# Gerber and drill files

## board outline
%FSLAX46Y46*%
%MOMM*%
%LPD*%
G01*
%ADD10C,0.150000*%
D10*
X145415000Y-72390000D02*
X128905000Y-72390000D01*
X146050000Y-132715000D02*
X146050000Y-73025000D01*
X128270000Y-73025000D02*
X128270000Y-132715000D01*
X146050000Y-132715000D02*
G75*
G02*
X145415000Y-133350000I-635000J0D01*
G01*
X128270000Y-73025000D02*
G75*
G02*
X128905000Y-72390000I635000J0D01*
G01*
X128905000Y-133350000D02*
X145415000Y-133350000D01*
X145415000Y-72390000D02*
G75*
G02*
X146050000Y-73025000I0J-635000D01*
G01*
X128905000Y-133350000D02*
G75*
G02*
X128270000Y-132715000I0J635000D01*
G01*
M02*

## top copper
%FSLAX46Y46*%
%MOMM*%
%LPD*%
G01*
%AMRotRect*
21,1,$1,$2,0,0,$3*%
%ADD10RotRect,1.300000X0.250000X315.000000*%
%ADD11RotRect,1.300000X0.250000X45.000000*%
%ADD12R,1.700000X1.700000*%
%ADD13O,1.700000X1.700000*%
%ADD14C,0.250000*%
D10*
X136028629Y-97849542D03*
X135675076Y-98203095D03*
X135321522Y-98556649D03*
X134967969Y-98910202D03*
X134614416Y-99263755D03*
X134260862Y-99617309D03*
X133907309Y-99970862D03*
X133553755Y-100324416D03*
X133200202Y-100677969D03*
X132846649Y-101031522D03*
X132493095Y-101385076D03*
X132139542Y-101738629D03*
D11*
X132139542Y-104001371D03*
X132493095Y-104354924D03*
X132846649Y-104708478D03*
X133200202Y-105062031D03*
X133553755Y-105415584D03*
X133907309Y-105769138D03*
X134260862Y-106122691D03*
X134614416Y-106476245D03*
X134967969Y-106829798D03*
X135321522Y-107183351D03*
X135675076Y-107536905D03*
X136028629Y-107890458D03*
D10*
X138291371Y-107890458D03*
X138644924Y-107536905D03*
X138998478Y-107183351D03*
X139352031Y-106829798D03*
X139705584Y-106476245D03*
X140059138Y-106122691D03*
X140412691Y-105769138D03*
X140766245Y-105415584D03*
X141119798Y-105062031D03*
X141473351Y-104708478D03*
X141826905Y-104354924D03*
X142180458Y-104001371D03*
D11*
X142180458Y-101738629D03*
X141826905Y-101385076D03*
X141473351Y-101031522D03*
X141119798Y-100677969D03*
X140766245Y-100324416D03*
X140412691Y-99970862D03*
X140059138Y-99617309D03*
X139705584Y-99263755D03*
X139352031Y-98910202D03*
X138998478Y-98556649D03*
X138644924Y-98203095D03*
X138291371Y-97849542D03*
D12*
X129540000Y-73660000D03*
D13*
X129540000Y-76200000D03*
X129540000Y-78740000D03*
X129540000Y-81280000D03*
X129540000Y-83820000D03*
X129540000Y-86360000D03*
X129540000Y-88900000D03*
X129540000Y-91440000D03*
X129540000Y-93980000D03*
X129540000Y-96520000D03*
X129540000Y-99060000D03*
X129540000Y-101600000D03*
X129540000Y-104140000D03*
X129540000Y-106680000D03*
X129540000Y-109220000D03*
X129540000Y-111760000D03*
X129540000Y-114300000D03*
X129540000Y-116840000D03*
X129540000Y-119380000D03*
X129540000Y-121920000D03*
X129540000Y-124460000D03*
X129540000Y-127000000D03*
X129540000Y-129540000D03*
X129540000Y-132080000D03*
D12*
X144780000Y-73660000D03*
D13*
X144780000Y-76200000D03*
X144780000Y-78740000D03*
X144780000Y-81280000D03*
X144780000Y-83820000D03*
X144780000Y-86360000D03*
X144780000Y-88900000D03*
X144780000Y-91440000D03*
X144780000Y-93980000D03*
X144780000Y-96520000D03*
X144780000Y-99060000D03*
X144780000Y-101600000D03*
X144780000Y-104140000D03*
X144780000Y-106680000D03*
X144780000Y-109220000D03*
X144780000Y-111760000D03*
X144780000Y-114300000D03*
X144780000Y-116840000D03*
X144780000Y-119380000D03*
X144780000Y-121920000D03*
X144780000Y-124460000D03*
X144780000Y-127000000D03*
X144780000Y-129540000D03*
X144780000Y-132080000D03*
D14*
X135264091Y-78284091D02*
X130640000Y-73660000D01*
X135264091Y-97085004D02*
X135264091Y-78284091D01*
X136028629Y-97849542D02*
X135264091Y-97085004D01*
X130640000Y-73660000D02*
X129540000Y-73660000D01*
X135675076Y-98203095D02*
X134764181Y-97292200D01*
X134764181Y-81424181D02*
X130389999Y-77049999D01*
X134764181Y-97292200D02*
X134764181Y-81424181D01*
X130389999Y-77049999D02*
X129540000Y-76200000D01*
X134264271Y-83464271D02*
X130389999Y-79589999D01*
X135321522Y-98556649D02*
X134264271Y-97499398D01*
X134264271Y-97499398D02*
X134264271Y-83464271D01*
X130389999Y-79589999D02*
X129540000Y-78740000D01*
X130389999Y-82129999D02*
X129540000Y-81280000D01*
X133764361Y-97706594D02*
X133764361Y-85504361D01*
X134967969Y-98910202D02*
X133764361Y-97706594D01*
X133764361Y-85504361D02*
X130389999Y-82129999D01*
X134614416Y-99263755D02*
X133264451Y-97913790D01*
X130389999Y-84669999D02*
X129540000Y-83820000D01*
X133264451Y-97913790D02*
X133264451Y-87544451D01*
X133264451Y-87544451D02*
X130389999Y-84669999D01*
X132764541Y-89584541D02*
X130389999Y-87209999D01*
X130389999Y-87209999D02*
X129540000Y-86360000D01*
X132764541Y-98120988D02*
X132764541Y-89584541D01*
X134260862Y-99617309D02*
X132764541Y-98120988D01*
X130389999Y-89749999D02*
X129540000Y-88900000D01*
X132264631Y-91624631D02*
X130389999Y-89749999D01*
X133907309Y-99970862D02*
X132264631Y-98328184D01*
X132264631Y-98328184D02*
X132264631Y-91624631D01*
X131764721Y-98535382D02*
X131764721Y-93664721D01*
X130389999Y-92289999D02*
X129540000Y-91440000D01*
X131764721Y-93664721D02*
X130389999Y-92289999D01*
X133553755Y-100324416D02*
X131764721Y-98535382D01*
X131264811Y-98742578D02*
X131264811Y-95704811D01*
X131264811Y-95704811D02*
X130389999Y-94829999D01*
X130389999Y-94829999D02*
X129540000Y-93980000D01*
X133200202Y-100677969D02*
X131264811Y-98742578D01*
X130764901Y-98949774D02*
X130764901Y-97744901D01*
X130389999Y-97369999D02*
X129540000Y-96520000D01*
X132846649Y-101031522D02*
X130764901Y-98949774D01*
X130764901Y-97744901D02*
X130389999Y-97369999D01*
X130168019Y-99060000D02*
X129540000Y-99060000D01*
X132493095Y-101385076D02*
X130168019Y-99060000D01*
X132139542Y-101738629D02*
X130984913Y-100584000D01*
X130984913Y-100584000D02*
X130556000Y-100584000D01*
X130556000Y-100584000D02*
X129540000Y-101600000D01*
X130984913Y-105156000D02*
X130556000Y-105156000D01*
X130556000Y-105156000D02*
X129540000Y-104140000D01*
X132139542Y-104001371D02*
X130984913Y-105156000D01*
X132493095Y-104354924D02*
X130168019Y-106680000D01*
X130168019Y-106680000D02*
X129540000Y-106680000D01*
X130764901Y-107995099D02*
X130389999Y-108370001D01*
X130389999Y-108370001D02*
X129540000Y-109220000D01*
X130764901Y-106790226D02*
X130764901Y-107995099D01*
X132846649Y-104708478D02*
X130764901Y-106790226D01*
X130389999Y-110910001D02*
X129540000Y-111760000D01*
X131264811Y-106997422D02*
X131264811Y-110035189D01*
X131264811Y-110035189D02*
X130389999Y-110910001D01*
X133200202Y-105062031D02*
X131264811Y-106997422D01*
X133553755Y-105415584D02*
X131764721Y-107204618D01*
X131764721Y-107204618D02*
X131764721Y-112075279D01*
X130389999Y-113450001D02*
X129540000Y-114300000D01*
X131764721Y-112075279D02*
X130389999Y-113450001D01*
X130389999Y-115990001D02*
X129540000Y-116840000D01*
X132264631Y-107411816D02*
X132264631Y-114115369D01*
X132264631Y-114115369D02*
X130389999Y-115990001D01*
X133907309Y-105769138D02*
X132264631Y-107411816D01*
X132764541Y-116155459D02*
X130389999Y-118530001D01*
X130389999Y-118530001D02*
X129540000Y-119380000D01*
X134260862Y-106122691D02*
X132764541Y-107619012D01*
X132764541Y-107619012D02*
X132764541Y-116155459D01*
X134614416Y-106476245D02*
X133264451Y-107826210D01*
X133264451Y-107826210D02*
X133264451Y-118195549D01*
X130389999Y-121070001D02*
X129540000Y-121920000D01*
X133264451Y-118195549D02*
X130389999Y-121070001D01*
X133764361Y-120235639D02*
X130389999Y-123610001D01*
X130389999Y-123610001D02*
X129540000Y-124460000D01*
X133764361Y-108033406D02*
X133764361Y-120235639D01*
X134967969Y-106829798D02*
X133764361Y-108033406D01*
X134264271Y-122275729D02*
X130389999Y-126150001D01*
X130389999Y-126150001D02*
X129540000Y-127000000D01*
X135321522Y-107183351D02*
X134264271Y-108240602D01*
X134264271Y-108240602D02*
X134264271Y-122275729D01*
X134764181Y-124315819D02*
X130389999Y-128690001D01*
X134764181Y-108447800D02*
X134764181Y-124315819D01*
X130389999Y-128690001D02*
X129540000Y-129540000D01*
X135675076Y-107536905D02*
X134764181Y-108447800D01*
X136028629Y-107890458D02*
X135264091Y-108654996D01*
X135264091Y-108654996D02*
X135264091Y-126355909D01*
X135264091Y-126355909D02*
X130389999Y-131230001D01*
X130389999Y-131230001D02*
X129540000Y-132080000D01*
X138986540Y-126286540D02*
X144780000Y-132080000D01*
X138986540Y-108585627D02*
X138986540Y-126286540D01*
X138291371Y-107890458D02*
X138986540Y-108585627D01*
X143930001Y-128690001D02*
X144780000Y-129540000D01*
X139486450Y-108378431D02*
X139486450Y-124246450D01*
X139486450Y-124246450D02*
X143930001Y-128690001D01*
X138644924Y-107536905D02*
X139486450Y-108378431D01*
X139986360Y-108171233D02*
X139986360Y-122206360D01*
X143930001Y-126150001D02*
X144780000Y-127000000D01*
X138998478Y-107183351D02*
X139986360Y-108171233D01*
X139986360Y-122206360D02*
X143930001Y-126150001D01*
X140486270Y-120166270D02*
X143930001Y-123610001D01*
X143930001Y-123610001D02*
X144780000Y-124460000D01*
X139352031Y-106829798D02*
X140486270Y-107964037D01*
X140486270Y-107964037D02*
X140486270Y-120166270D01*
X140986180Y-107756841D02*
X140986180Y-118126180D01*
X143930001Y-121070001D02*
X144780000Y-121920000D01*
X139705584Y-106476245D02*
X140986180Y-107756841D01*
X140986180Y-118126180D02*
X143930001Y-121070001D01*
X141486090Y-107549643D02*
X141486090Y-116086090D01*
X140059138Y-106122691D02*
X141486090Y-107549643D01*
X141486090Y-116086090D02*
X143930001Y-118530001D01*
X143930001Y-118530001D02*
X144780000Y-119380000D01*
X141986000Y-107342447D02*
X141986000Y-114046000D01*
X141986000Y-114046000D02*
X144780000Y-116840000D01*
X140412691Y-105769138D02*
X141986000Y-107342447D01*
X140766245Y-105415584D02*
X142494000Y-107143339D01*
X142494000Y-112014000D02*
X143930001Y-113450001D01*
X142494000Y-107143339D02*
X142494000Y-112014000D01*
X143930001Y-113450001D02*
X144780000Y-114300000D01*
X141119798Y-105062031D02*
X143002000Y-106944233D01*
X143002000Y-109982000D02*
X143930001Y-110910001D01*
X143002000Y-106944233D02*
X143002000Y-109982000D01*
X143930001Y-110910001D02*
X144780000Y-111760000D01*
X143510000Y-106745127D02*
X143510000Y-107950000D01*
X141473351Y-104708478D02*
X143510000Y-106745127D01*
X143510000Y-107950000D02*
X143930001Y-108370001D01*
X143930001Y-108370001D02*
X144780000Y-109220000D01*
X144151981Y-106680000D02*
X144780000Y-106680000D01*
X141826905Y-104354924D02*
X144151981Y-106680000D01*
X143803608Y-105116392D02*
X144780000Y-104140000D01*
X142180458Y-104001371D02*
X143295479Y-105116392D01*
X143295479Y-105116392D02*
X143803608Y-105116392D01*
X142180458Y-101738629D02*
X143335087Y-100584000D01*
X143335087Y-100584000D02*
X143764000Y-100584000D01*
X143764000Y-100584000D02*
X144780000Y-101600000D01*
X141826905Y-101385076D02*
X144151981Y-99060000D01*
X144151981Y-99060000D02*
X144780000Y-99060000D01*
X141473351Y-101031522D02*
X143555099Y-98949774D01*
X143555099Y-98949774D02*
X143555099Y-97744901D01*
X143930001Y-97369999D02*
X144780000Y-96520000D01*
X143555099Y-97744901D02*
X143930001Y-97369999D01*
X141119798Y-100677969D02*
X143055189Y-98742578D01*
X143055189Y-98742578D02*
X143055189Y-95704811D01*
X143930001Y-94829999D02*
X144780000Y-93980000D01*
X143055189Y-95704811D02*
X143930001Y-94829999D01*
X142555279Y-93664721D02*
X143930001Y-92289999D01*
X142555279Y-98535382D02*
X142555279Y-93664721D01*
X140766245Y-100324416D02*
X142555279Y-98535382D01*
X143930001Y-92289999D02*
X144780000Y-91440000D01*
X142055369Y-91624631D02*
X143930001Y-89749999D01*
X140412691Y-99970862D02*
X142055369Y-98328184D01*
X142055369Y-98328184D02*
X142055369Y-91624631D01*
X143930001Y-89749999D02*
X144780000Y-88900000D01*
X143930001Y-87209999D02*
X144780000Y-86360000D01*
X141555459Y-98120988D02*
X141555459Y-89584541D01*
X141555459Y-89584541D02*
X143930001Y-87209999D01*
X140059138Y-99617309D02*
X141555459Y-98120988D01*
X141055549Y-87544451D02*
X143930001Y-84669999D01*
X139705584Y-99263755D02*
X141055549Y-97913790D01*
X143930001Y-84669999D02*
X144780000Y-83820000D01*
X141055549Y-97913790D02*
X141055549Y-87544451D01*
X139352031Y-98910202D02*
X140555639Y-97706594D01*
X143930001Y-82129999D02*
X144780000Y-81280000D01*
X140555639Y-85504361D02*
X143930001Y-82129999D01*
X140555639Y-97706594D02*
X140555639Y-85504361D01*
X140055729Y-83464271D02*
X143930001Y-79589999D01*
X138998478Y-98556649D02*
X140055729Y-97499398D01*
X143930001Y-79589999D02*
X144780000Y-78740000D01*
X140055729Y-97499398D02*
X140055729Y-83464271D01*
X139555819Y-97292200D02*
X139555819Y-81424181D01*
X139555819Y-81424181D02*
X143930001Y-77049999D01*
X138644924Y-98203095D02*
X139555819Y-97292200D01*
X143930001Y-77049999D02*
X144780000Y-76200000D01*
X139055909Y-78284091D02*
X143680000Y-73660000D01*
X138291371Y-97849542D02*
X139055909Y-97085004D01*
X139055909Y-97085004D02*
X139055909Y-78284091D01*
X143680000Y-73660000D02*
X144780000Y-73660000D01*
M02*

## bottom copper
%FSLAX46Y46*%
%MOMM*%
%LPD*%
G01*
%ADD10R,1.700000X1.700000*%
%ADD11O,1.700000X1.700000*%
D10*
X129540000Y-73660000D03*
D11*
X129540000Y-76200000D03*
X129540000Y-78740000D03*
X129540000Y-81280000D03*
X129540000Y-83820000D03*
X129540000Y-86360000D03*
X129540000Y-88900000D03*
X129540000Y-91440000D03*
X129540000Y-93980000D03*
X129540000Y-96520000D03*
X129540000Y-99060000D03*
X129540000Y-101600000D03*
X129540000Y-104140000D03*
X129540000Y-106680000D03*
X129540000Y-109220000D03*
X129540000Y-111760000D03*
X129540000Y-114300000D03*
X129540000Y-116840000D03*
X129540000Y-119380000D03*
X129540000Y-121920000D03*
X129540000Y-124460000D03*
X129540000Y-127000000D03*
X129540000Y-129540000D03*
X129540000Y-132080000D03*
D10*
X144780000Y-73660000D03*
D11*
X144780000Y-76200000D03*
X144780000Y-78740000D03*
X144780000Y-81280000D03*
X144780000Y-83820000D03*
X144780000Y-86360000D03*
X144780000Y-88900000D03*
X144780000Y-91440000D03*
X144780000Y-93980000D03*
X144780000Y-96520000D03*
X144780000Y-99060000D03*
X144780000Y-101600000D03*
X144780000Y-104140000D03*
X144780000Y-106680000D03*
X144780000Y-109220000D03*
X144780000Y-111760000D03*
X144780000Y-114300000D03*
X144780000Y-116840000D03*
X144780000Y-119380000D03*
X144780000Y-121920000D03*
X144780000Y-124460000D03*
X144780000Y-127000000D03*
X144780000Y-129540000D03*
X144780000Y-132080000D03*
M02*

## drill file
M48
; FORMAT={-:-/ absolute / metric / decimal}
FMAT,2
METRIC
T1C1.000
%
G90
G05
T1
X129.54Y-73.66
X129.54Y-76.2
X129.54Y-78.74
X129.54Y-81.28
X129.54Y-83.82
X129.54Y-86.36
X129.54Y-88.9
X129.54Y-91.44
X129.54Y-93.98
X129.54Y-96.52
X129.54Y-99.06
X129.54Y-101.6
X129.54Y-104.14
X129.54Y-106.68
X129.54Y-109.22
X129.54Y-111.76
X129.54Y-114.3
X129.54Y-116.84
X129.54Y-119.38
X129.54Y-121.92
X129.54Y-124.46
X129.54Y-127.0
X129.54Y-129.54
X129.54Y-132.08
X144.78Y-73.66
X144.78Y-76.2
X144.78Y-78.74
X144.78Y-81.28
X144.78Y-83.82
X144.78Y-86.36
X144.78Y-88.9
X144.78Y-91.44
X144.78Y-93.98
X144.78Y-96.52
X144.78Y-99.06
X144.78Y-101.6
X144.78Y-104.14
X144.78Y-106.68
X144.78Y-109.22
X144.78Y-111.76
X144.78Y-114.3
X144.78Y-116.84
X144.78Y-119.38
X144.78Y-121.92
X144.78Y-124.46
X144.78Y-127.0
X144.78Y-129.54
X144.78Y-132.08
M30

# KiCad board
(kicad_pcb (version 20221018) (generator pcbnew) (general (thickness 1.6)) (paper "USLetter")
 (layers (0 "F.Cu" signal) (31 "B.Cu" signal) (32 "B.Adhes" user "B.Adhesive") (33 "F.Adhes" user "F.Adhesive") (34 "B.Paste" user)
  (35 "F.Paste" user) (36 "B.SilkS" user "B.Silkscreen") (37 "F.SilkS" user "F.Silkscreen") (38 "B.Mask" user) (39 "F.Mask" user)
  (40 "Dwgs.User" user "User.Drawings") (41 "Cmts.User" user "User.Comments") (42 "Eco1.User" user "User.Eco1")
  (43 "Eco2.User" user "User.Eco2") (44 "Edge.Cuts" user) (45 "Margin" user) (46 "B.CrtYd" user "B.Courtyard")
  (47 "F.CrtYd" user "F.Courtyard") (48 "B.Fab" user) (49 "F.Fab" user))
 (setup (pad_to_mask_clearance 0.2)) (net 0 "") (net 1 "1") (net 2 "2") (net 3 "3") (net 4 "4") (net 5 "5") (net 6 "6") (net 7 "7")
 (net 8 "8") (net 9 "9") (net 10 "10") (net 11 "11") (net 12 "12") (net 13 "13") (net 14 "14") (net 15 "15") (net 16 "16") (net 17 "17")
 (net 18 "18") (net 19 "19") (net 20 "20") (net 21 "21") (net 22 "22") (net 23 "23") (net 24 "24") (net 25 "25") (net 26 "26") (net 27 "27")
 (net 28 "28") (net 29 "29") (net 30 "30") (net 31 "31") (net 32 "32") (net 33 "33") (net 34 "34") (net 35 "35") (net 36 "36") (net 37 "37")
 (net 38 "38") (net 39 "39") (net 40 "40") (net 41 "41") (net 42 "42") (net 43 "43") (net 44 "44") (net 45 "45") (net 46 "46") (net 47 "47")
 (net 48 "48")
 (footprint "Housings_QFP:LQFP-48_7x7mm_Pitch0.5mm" (layer "F.Cu") (at 137.16 102.87 -45)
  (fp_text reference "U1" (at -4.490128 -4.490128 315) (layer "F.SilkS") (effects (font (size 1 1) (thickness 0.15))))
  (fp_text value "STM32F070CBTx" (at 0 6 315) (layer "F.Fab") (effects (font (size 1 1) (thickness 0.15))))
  (pad "1" smd rect (at -4.35 -2.75 315) (size 1.3 0.25) (layers "F.Cu" "F.Paste" "F.Mask") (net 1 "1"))
  (pad "2" smd rect (at -4.35 -2.25 315) (size 1.3 0.25) (layers "F.Cu" "F.Paste" "F.Mask") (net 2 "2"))
  (pad "3" smd rect (at -4.35 -1.749999 315) (size 1.3 0.25) (layers "F.Cu" "F.Paste" "F.Mask") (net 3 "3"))
  (pad "4" smd rect (at -4.35 -1.25 315) (size 1.3 0.25) (layers "F.Cu" "F.Paste" "F.Mask") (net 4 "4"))
  (pad "5" smd rect (at -4.35 -0.750001 315) (size 1.3 0.25) (layers "F.Cu" "F.Paste" "F.Mask") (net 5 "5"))
  (pad "6" smd rect (at -4.35 -0.25 315) (size 1.3 0.25) (layers "F.Cu" "F.Paste" "F.Mask") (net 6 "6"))
  (pad "7" smd rect (at -4.35 0.25 315) (size 1.3 0.25) (layers "F.Cu" "F.Paste" "F.Mask") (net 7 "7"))
  (pad "8" smd rect (at -4.35 0.750001 315) (size 1.3 0.25) (layers "F.Cu" "F.Paste" "F.Mask") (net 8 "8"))
  (pad "9" smd rect (at -4.35 1.25 315) (size 1.3 0.25) (layers "F.Cu" "F.Paste" "F.Mask") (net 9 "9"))
  (pad "10" smd rect (at -4.35 1.749999 315) (size 1.3 0.25) (layers "F.Cu" "F.Paste" "F.Mask") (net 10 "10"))
  (pad "11" smd rect (at -4.35 2.25 315) (size 1.3 0.25) (layers "F.Cu" "F.Paste" "F.Mask") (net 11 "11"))
  (pad "12" smd rect (at -4.35 2.75 315) (size 1.3 0.25) (layers "F.Cu" "F.Paste" "F.Mask") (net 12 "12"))
  (pad "13" smd rect (at -2.75 4.35 45) (size 1.3 0.25) (layers "F.Cu" "F.Paste" "F.Mask") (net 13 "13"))
  (pad "14" smd rect (at -2.25 4.35 45) (size 1.3 0.25) (layers "F.Cu" "F.Paste" "F.Mask") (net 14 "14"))
  (pad "15" smd rect (at -1.749999 4.35 45) (size 1.3 0.25) (layers "F.Cu" "F.Paste" "F.Mask") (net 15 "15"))
  (pad "16" smd rect (at -1.25 4.35 45) (size 1.3 0.25) (layers "F.Cu" "F.Paste" "F.Mask") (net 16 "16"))
  (pad "17" smd rect (at -0.750001 4.35 45) (size 1.3 0.25) (layers "F.Cu" "F.Paste" "F.Mask") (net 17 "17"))
  (pad "18" smd rect (at -0.25 4.35 45) (size 1.3 0.25) (layers "F.Cu" "F.Paste" "F.Mask") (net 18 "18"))
  (pad "19" smd rect (at 0.25 4.35 45) (size 1.3 0.25) (layers "F.Cu" "F.Paste" "F.Mask") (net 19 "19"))
  (pad "20" smd rect (at 0.750001 4.35 45) (size 1.3 0.25) (layers "F.Cu" "F.Paste" "F.Mask") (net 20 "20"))
  (pad "21" smd rect (at 1.25 4.35 45) (size 1.3 0.25) (layers "F.Cu" "F.Paste" "F.Mask") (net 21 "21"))
  (pad "22" smd rect (at 1.749999 4.35 45) (size 1.3 0.25) (layers "F.Cu" "F.Paste" "F.Mask") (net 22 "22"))
  (pad "23" smd rect (at 2.25 4.35 45) (size 1.3 0.25) (layers "F.Cu" "F.Paste" "F.Mask") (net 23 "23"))
  (pad "24" smd rect (at 2.75 4.35 45) (size 1.3 0.25) (layers "F.Cu" "F.Paste" "F.Mask") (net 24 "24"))
  (pad "25" smd rect (at 4.35 2.75 315) (size 1.3 0.25) (layers "F.Cu" "F.Paste" "F.Mask") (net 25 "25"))
  (pad "26" smd rect (at 4.35 2.25 315) (size 1.3 0.25) (layers "F.Cu" "F.Paste" "F.Mask") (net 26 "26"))
  (pad "27" smd rect (at 4.35 1.749999 315) (size 1.3 0.25) (layers "F.Cu" "F.Paste" "F.Mask") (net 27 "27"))
  (pad "28" smd rect (at 4.35 1.25 315) (size 1.3 0.25) (layers "F.Cu" "F.Paste" "F.Mask") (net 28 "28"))
  (pad "29" smd rect (at 4.35 0.750001 315) (size 1.3 0.25) (layers "F.Cu" "F.Paste" "F.Mask") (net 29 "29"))
  (pad "30" smd rect (at 4.35 0.25 315) (size 1.3 0.25) (layers "F.Cu" "F.Paste" "F.Mask") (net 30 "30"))
  (pad "31" smd rect (at 4.35 -0.25 315) (size 1.3 0.25) (layers "F.Cu" "F.Paste" "F.Mask") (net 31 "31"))
  (pad "32" smd rect (at 4.35 -0.750001 315) (size 1.3 0.25) (layers "F.Cu" "F.Paste" "F.Mask") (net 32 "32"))
  (pad "33" smd rect (at 4.35 -1.25 315) (size 1.3 0.25) (layers "F.Cu" "F.Paste" "F.Mask") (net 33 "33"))
  (pad "34" smd rect (at 4.35 -1.749999 315) (size 1.3 0.25) (layers "F.Cu" "F.Paste" "F.Mask") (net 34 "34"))
  (pad "35" smd rect (at 4.35 -2.25 315) (size 1.3 0.25) (layers "F.Cu" "F.Paste" "F.Mask") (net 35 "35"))
  (pad "36" smd rect (at 4.35 -2.75 315) (size 1.3 0.25) (layers "F.Cu" "F.Paste" "F.Mask") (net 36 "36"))
  (pad "37" smd rect (at 2.75 -4.35 45) (size 1.3 0.25) (layers "F.Cu" "F.Paste" "F.Mask") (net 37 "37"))
  (pad "38" smd rect (at 2.25 -4.35 45) (size 1.3 0.25) (layers "F.Cu" "F.Paste" "F.Mask") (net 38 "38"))
  (pad "39" smd rect (at 1.749999 -4.35 45) (size 1.3 0.25) (layers "F.Cu" "F.Paste" "F.Mask") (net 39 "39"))
  (pad "40" smd rect (at 1.25 -4.35 45) (size 1.3 0.25) (layers "F.Cu" "F.Paste" "F.Mask") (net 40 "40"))
  (pad "41" smd rect (at 0.750001 -4.35 45) (size 1.3 0.25) (layers "F.Cu" "F.Paste" "F.Mask") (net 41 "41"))
  (pad "42" smd rect (at 0.25 -4.35 45) (size 1.3 0.25) (layers "F.Cu" "F.Paste" "F.Mask") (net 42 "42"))
  (pad "43" smd rect (at -0.25 -4.35 45) (size 1.3 0.25) (layers "F.Cu" "F.Paste" "F.Mask") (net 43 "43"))
  (pad "44" smd rect (at -0.750001 -4.35 45) (size 1.3 0.25) (layers "F.Cu" "F.Paste" "F.Mask") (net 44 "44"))
  (pad "45" smd rect (at -1.25 -4.35 45) (size 1.3 0.25) (layers "F.Cu" "F.Paste" "F.Mask") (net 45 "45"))
  (pad "46" smd rect (at -1.749999 -4.35 45) (size 1.3 0.25) (layers "F.Cu" "F.Paste" "F.Mask") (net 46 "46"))
  (pad "47" smd rect (at -2.25 -4.35 45) (size 1.3 0.25) (layers "F.Cu" "F.Paste" "F.Mask") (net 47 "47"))
  (pad "48" smd rect (at -2.75 -4.35 45) (size 1.3 0.25) (layers "F.Cu" "F.Paste" "F.Mask") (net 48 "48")))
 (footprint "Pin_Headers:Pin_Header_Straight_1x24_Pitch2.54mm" (layer "B.Cu") (at 129.54 73.66 180)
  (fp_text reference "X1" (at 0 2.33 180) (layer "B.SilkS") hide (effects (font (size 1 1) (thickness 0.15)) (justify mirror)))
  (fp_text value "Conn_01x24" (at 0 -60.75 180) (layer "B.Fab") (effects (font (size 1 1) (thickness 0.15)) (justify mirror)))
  (pad "1" thru_hole rect (at 0 0 180) (size 1.7 1.7) (drill 1) (layers "*.Cu" "*.Mask") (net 1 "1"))
  (pad "2" thru_hole oval (at 0 -2.54 180) (size 1.7 1.7) (drill 1) (layers "*.Cu" "*.Mask") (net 2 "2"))
  (pad "3" thru_hole oval (at 0 -5.08 180) (size 1.7 1.7) (drill 1) (layers "*.Cu" "*.Mask") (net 3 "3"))
  (pad "4" thru_hole oval (at 0 -7.62 180) (size 1.7 1.7) (drill 1) (layers "*.Cu" "*.Mask") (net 4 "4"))
  (pad "5" thru_hole oval (at 0 -10.16 180) (size 1.7 1.7) (drill 1) (layers "*.Cu" "*.Mask") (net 5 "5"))
  (pad "6" thru_hole oval (at 0 -12.7 180) (size 1.7 1.7) (drill 1) (layers "*.Cu" "*.Mask") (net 6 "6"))
  (pad "7" thru_hole oval (at 0 -15.24 180) (size 1.7 1.7) (drill 1) (layers "*.Cu" "*.Mask") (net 7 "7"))
  (pad "8" thru_hole oval (at 0 -17.78 180) (size 1.7 1.7) (drill 1) (layers "*.Cu" "*.Mask") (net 8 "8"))
  (pad "9" thru_hole oval (at 0 -20.32 180) (size 1.7 1.7) (drill 1) (layers "*.Cu" "*.Mask") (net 9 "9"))
  (pad "10" thru_hole oval (at 0 -22.86 180) (size 1.7 1.7) (drill 1) (layers "*.Cu" "*.Mask") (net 10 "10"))
  (pad "11" thru_hole oval (at 0 -25.4 180) (size 1.7 1.7) (drill 1) (layers "*.Cu" "*.Mask") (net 11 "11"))
  (pad "12" thru_hole oval (at 0 -27.94 180) (size 1.7 1.7) (drill 1) (layers "*.Cu" "*.Mask") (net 12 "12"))
  (pad "13" thru_hole oval (at 0 -30.48 180) (size 1.7 1.7) (drill 1) (layers "*.Cu" "*.Mask") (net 13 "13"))
  (pad "14" thru_hole oval (at 0 -33.02 180) (size 1.7 1.7) (drill 1) (layers "*.Cu" "*.Mask") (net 14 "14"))
  (pad "15" thru_hole oval (at 0 -35.56 180) (size 1.7 1.7) (drill 1) (layers "*.Cu" "*.Mask") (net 15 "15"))
  (pad "16" thru_hole oval (at 0 -38.1 180) (size 1.7 1.7) (drill 1) (layers "*.Cu" "*.Mask") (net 16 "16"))
  (pad "17" thru_hole oval (at 0 -40.64 180) (size 1.7 1.7) (drill 1) (layers "*.Cu" "*.Mask") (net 17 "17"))
  (pad "18" thru_hole oval (at 0 -43.18 180) (size 1.7 1.7) (drill 1) (layers "*.Cu" "*.Mask") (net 18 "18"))
  (pad "19" thru_hole oval (at 0 -45.72 180) (size 1.7 1.7) (drill 1) (layers "*.Cu" "*.Mask") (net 19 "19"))
  (pad "20" thru_hole oval (at 0 -48.26 180) (size 1.7 1.7) (drill 1) (layers "*.Cu" "*.Mask") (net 20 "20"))
  (pad "21" thru_hole oval (at 0 -50.8 180) (size 1.7 1.7) (drill 1) (layers "*.Cu" "*.Mask") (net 21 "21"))
  (pad "22" thru_hole oval (at 0 -53.34 180) (size 1.7 1.7) (drill 1) (layers "*.Cu" "*.Mask") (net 22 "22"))
  (pad "23" thru_hole oval (at 0 -55.88 180) (size 1.7 1.7) (drill 1) (layers "*.Cu" "*.Mask") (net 23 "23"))
  (pad "24" thru_hole oval (at 0 -58.42 180) (size 1.7 1.7) (drill 1) (layers "*.Cu" "*.Mask") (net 24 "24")))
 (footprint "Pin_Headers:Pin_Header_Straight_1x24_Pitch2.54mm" (layer "B.Cu") (at 144.78 73.66 180)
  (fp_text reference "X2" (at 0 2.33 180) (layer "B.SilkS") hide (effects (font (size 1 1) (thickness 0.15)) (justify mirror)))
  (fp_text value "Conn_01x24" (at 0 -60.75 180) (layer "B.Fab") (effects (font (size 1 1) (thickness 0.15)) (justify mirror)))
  (pad "1" thru_hole rect (at 0 0 180) (size 1.7 1.7) (drill 1) (layers "*.Cu" "*.Mask") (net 48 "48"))
  (pad "2" thru_hole oval (at 0 -2.54 180) (size 1.7 1.7) (drill 1) (layers "*.Cu" "*.Mask") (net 47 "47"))
  (pad "3" thru_hole oval (at 0 -5.08 180) (size 1.7 1.7) (drill 1) (layers "*.Cu" "*.Mask") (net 46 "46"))
  (pad "4" thru_hole oval (at 0 -7.62 180) (size 1.7 1.7) (drill 1) (layers "*.Cu" "*.Mask") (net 45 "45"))
  (pad "5" thru_hole oval (at 0 -10.16 180) (size 1.7 1.7) (drill 1) (layers "*.Cu" "*.Mask") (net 44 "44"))
  (pad "6" thru_hole oval (at 0 -12.7 180) (size 1.7 1.7) (drill 1) (layers "*.Cu" "*.Mask") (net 43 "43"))
  (pad "7" thru_hole oval (at 0 -15.24 180) (size 1.7 1.7) (drill 1) (layers "*.Cu" "*.Mask") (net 42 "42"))
  (pad "8" thru_hole oval (at 0 -17.78 180) (size 1.7 1.7) (drill 1) (layers "*.Cu" "*.Mask") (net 41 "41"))
  (pad "9" thru_hole oval (at 0 -20.32 180) (size 1.7 1.7) (drill 1) (layers "*.Cu" "*.Mask") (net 40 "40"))
  (pad "10" thru_hole oval (at 0 -22.86 180) (size 1.7 1.7) (drill 1) (layers "*.Cu" "*.Mask") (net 39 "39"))
  (pad "11" thru_hole oval (at 0 -25.4 180) (size 1.7 1.7) (drill 1) (layers "*.Cu" "*.Mask") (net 38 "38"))
  (pad "12" thru_hole oval (at 0 -27.94 180) (size 1.7 1.7) (drill 1) (layers "*.Cu" "*.Mask") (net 37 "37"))
  (pad "13" thru_hole oval (at 0 -30.48 180) (size 1.7 1.7) (drill 1) (layers "*.Cu" "*.Mask") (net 36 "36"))
  (pad "14" thru_hole oval (at 0 -33.02 180) (size 1.7 1.7) (drill 1) (layers "*.Cu" "*.Mask") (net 35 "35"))
  (pad "15" thru_hole oval (at 0 -35.56 180) (size 1.7 1.7) (drill 1) (layers "*.Cu" "*.Mask") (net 34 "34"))
  (pad "16" thru_hole oval (at 0 -38.1 180) (size 1.7 1.7) (drill 1) (layers "*.Cu" "*.Mask") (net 33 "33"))
  (pad "17" thru_hole oval (at 0 -40.64 180) (size 1.7 1.7) (drill 1) (layers "*.Cu" "*.Mask") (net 32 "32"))
  (pad "18" thru_hole oval (at 0 -43.18 180) (size 1.7 1.7) (drill 1) (layers "*.Cu" "*.Mask") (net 31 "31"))
  (pad "19" thru_hole oval (at 0 -45.72 180) (size 1.7 1.7) (drill 1) (layers "*.Cu" "*.Mask") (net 30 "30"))
  (pad "20" thru_hole oval (at 0 -48.26 180) (size 1.7 1.7) (drill 1) (layers "*.Cu" "*.Mask") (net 29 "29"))
  (pad "21" thru_hole oval (at 0 -50.8 180) (size 1.7 1.7) (drill 1) (layers "*.Cu" "*.Mask") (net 28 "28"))
  (pad "22" thru_hole oval (at 0 -53.34 180) (size 1.7 1.7) (drill 1) (layers "*.Cu" "*.Mask") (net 27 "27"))
  (pad "23" thru_hole oval (at 0 -55.88 180) (size 1.7 1.7) (drill 1) (layers "*.Cu" "*.Mask") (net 26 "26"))
  (pad "24" thru_hole oval (at 0 -58.42 180) (size 1.7 1.7) (drill 1) (layers "*.Cu" "*.Mask") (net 25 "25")))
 (gr_line (start 145.415 72.39) (end 128.905 72.39) (stroke (width 0.15) (type solid)) (layer "Edge.Cuts"))
 (gr_line (start 146.05 132.715) (end 146.05 73.025) (stroke (width 0.15) (type solid)) (layer "Edge.Cuts"))
 (gr_line (start 128.27 73.025) (end 128.27 132.715) (stroke (width 0.15) (type solid)) (layer "Edge.Cuts"))
 (gr_arc (start 146.05 132.715) (mid 145.864013 133.164013) (end 145.415 133.35) (stroke (width 0.15) (type solid)) (layer "Edge.Cuts"))
 (gr_arc (start 128.27 73.025) (mid 128.455987 72.575987) (end 128.905 72.39) (stroke (width 0.15) (type solid)) (layer "Edge.Cuts"))
 (gr_line (start 128.905 133.35) (end 145.415 133.35) (stroke (width 0.15) (type solid)) (layer "Edge.Cuts"))
 (gr_arc (start 145.415 72.39) (mid 145.864013 72.575987) (end 146.05 73.025) (stroke (width 0.15) (type solid)) (layer "Edge.Cuts"))
 (gr_arc (start 128.905 133.35) (mid 128.455987 133.164013) (end 128.27 132.715) (stroke (width 0.15) (type solid)) (layer "Edge.Cuts"))
 (segment (start 135.264091 78.284091) (end 130.64 73.66) (width 0.25) (layer "F.Cu") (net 1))
 (segment (start 135.264091 97.085004) (end 135.264091 78.284091) (width 0.25) (layer "F.Cu") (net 1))
 (segment (start 136.028629 97.849542) (end 135.264091 97.085004) (width 0.25) (layer "F.Cu") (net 1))
 (segment (start 130.64 73.66) (end 129.54 73.66) (width 0.25) (layer "F.Cu") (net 1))
 (segment (start 135.675076 98.203095) (end 134.764181 97.2922) (width 0.25) (layer "F.Cu") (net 2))
 (segment (start 134.764181 81.424181) (end 130.389999 77.049999) (width 0.25) (layer "F.Cu") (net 2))
 (segment (start 134.764181 97.2922) (end 134.764181 81.424181) (width 0.25) (layer "F.Cu") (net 2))
 (segment (start 130.389999 77.049999) (end 129.54 76.2) (width 0.25) (layer "F.Cu") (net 2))
 (segment (start 134.264271 83.464271) (end 130.389999 79.589999) (width 0.25) (layer "F.Cu") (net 3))
 (segment (start 135.321522 98.556649) (end 134.264271 97.499398) (width 0.25) (layer "F.Cu") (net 3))
 (segment (start 134.264271 97.499398) (end 134.264271 83.464271) (width 0.25) (layer "F.Cu") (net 3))
 (segment (start 130.389999 79.589999) (end 129.54 78.74) (width 0.25) (layer "F.Cu") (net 3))
 (segment (start 130.389999 82.129999) (end 129.54 81.28) (width 0.25) (layer "F.Cu") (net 4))
 (segment (start 133.764361 97.706594) (end 133.764361 85.504361) (width 0.25) (layer "F.Cu") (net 4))
 (segment (start 134.967969 98.910202) (end 133.764361 97.706594) (width 0.25) (layer "F.Cu") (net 4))
 (segment (start 133.764361 85.504361) (end 130.389999 82.129999) (width 0.25) (layer "F.Cu") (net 4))
 (segment (start 134.614416 99.263755) (end 133.264451 97.91379) (width 0.25) (layer "F.Cu") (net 5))
 (segment (start 130.389999 84.669999) (end 129.54 83.82) (width 0.25) (layer "F.Cu") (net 5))
 (segment (start 133.264451 97.91379) (end 133.264451 87.544451) (width 0.25) (layer "F.Cu") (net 5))
 (segment (start 133.264451 87.544451) (end 130.389999 84.669999) (width 0.25) (layer "F.Cu") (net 5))
 (segment (start 132.764541 89.584541) (end 130.389999 87.209999) (width 0.25) (layer "F.Cu") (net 6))
 (segment (start 130.389999 87.209999) (end 129.54 86.36) (width 0.25) (layer "F.Cu") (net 6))
 (segment (start 132.764541 98.120988) (end 132.764541 89.584541) (width 0.25) (layer "F.Cu") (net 6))
 (segment (start 134.260862 99.617309) (end 132.764541 98.120988) (width 0.25) (layer "F.Cu") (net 6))
 (segment (start 130.389999 89.749999) (end 129.54 88.9) (width 0.25) (layer "F.Cu") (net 7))
 (segment (start 132.264631 91.624631) (end 130.389999 89.749999) (width 0.25) (layer "F.Cu") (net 7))
 (segment (start 133.907309 99.970862) (end 132.264631 98.328184) (width 0.25) (layer "F.Cu") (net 7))
 (segment (start 132.264631 98.328184) (end 132.264631 91.624631) (width 0.25) (layer "F.Cu") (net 7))
 (segment (start 131.764721 98.535382) (end 131.764721 93.664721) (width 0.25) (layer "F.Cu") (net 8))
 (segment (start 130.389999 92.289999) (end 129.54 91.44) (width 0.25) (layer "F.Cu") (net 8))
 (segment (start 131.764721 93.664721) (end 130.389999 92.289999) (width 0.25) (layer "F.Cu") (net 8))
 (segment (start 133.553755 100.324416) (end 131.764721 98.535382) (width 0.25) (layer "F.Cu") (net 8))
 (segment (start 131.264811 98.742578) (end 131.264811 95.704811) (width 0.25) (layer "F.Cu") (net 9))
 (segment (start 131.264811 95.704811) (end 130.389999 94.829999) (width 0.25) (layer "F.Cu") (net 9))
 (segment (start 130.389999 94.829999) (end 129.54 93.98) (width 0.25) (layer "F.Cu") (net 9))
 (segment (start 133.200202 100.677969) (end 131.264811 98.742578) (width 0.25) (layer "F.Cu") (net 9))
 (segment (start 130.764901 98.949774) (end 130.764901 97.744901) (width 0.25) (layer "F.Cu") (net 10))
 (segment (start 130.389999 97.369999) (end 129.54 96.52) (width 0.25) (layer "F.Cu") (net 10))
 (segment (start 132.846649 101.031522) (end 130.764901 98.949774) (width 0.25) (layer "F.Cu") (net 10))
 (segment (start 130.764901 97.744901) (end 130.389999 97.369999) (width 0.25) (layer "F.Cu") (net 10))
 (segment (start 130.168019 99.06) (end 129.54 99.06) (width 0.25) (layer "F.Cu") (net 11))
 (segment (start 132.493095 101.385076) (end 130.168019 99.06) (width 0.25) (layer "F.Cu") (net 11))
 (segment (start 132.139542 101.738629) (end 130.984913 100.584) (width 0.25) (layer "F.Cu") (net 12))
 (segment (start 130.984913 100.584) (end 130.556 100.584) (width 0.25) (layer "F.Cu") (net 12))
 (segment (start 130.556 100.584) (end 129.54 101.6) (width 0.25) (layer "F.Cu") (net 12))
 (segment (start 130.984913 105.156) (end 130.556 105.156) (width 0.25) (layer "F.Cu") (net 13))
 (segment (start 130.556 105.156) (end 129.54 104.14) (width 0.25) (layer "F.Cu") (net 13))
 (segment (start 132.139542 104.001371) (end 130.984913 105.156) (width 0.25) (layer "F.Cu") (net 13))
 (segment (start 132.493095 104.354924) (end 130.168019 106.68) (width 0.25) (layer "F.Cu") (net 14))
 (segment (start 130.168019 106.68) (end 129.54 106.68) (width 0.25) (layer "F.Cu") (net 14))
 (segment (start 130.764901 107.995099) (end 130.389999 108.370001) (width 0.25) (layer "F.Cu") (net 15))
 (segment (start 130.389999 108.370001) (end 129.54 109.22) (width 0.25) (layer "F.Cu") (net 15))
 (segment (start 130.764901 106.790226) (end 130.764901 107.995099) (width 0.25) (layer "F.Cu") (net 15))
 (segment (start 132.846649 104.708478) (end 130.764901 106.790226) (width 0.25) (layer "F.Cu") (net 15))
 (segment (start 130.389999 110.910001) (end 129.54 111.76) (width 0.25) (layer "F.Cu") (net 16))
 (segment (start 131.264811 106.997422) (end 131.264811 110.035189) (width 0.25) (layer "F.Cu") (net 16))
 (segment (start 131.264811 110.035189) (end 130.389999 110.910001) (width 0.25) (layer "F.Cu") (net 16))
 (segment (start 133.200202 105.062031) (end 131.264811 106.997422) (width 0.25) (layer "F.Cu") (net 16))
 (segment (start 133.553755 105.415584) (end 131.764721 107.204618) (width 0.25) (layer "F.Cu") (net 17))
 (segment (start 131.764721 107.204618) (end 131.764721 112.075279) (width 0.25) (layer "F.Cu") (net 17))
 (segment (start 130.389999 113.450001) (end 129.54 114.3) (width 0.25) (layer "F.Cu") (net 17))
 (segment (start 131.764721 112.075279) (end 130.389999 113.450001) (width 0.25) (layer "F.Cu") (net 17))
 (segment (start 130.389999 115.990001) (end 129.54 116.84) (width 0.25) (layer "F.Cu") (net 18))
 (segment (start 132.264631 107.411816) (end 132.264631 114.115369) (width 0.25) (layer "F.Cu") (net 18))
 (segment (start 132.264631 114.115369) (end 130.389999 115.990001) (width 0.25) (layer "F.Cu") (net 18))
 (segment (start 133.907309 105.769138) (end 132.264631 107.411816) (width 0.25) (layer "F.Cu") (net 18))
 (segment (start 132.764541 116.155459) (end 130.389999 118.530001) (width 0.25) (layer "F.Cu") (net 19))
 (segment (start 130.389999 118.530001) (end 129.54 119.38) (width 0.25) (layer "F.Cu") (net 19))
 (segment (start 134.260862 106.122691) (end 132.764541 107.619012) (width 0.25) (layer "F.Cu") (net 19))
 (segment (start 132.764541 107.619012) (end 132.764541 116.155459) (width 0.25) (layer "F.Cu") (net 19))
 (segment (start 134.614416 106.476245) (end 133.264451 107.82621) (width 0.25) (layer "F.Cu") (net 20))
 (segment (start 133.264451 107.82621) (end 133.264451 118.195549) (width 0.25) (layer "F.Cu") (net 20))
 (segment (start 130.389999 121.070001) (end 129.54 121.92) (width 0.25) (layer "F.Cu") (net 20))
 (segment (start 133.264451 118.195549) (end 130.389999 121.070001) (width 0.25) (layer "F.Cu") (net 20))
 (segment (start 133.764361 120.235639) (end 130.389999 123.610001) (width 0.25) (layer "F.Cu") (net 21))
 (segment (start 130.389999 123.610001) (end 129.54 124.46) (width 0.25) (layer "F.Cu") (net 21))
 (segment (start 133.764361 108.033406) (end 133.764361 120.235639) (width 0.25) (layer "F.Cu") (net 21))
 (segment (start 134.967969 106.829798) (end 133.764361 108.033406) (width 0.25) (layer "F.Cu") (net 21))
 (segment (start 134.264271 122.275729) (end 130.389999 126.150001) (width 0.25) (layer "F.Cu") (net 22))
 (segment (start 130.389999 126.150001) (end 129.54 127) (width 0.25) (layer "F.Cu") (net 22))
 (segment (start 135.321522 107.183351) (end 134.264271 108.240602) (width 0.25) (layer "F.Cu") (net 22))
 (segment (start 134.264271 108.240602) (end 134.264271 122.275729) (width 0.25) (layer "F.Cu") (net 22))
 (segment (start 134.764181 124.315819) (end 130.389999 128.690001) (width 0.25) (layer "F.Cu") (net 23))
 (segment (start 134.764181 108.4478) (end 134.764181 124.315819) (width 0.25) (layer "F.Cu") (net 23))
 (segment (start 130.389999 128.690001) (end 129.54 129.54) (width 0.25) (layer "F.Cu") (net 23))
 (segment (start 135.675076 107.536905) (end 134.764181 108.4478) (width 0.25) (layer "F.Cu") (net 23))
 (segment (start 136.028629 107.890458) (end 135.264091 108.654996) (width 0.25) (layer "F.Cu") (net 24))
 (segment (start 135.264091 108.654996) (end 135.264091 126.355909) (width 0.25) (layer "F.Cu") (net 24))
 (segment (start 135.264091 126.355909) (end 130.389999 131.230001) (width 0.25) (layer "F.Cu") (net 24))
 (segment (start 130.389999 131.230001) (end 129.54 132.08) (width 0.25) (layer "F.Cu") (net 24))
 (segment (start 138.98654 126.28654) (end 144.78 132.08) (width 0.25) (layer "F.Cu") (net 25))
 (segment (start 138.98654 108.585627) (end 138.98654 126.28654) (width 0.25) (layer "F.Cu") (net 25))
 (segment (start 138.291371 107.890458) (end 138.98654 108.585627) (width 0.25) (layer "F.Cu") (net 25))
 (segment (start 143.930001 128.690001) (end 144.78 129.54) (width 0.25) (layer "F.Cu") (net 26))
 (segment (start 139.48645 108.378431) (end 139.48645 124.24645) (width 0.25) (layer "F.Cu") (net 26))
 (segment (start 139.48645 124.24645) (end 143.930001 128.690001) (width 0.25) (layer "F.Cu") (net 26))
 (segment (start 138.644924 107.536905) (end 139.48645 108.378431) (width 0.25) (layer "F.Cu") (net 26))
 (segment (start 139.98636 108.171233) (end 139.98636 122.20636) (width 0.25) (layer "F.Cu") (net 27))
 (segment (start 143.930001 126.150001) (end 144.78 127) (width 0.25) (layer "F.Cu") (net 27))
 (segment (start 138.998478 107.183351) (end 139.98636 108.171233) (width 0.25) (layer "F.Cu") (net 27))
 (segment (start 139.98636 122.20636) (end 143.930001 126.150001) (width 0.25) (layer "F.Cu") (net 27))
 (segment (start 140.48627 120.16627) (end 143.930001 123.610001) (width 0.25) (layer "F.Cu") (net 28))
 (segment (start 143.930001 123.610001) (end 144.78 124.46) (width 0.25) (layer "F.Cu") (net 28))
 (segment (start 139.352031 106.829798) (end 140.48627 107.964037) (width 0.25) (layer "F.Cu") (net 28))
 (segment (start 140.48627 107.964037) (end 140.48627 120.16627) (width 0.25) (layer "F.Cu") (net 28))
 (segment (start 140.98618 107.756841) (end 140.98618 118.12618) (width 0.25) (layer "F.Cu") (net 29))
 (segment (start 143.930001 121.070001) (end 144.78 121.92) (width 0.25) (layer "F.Cu") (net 29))
 (segment (start 139.705584 106.476245) (end 140.98618 107.756841) (width 0.25) (layer "F.Cu") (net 29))
 (segment (start 140.98618 118.12618) (end 143.930001 121.070001) (width 0.25) (layer "F.Cu") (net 29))
 (segment (start 141.48609 107.549643) (end 141.48609 116.08609) (width 0.25) (layer "F.Cu") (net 30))
 (segment (start 140.059138 106.122691) (end 141.48609 107.549643) (width 0.25) (layer "F.Cu") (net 30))
 (segment (start 141.48609 116.08609) (end 143.930001 118.530001) (width 0.25) (layer "F.Cu") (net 30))
 (segment (start 143.930001 118.530001) (end 144.78 119.38) (width 0.25) (layer "F.Cu") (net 30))
 (segment (start 141.986 107.342447) (end 141.986 114.046) (width 0.25) (layer "F.Cu") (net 31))
 (segment (start 141.986 114.046) (end 144.78 116.84) (width 0.25) (layer "F.Cu") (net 31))
 (segment (start 140.412691 105.769138) (end 141.986 107.342447) (width 0.25) (layer "F.Cu") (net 31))
 (segment (start 140.766245 105.415584) (end 142.494 107.143339) (width 0.25) (layer "F.Cu") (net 32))
 (segment (start 142.494 112.014) (end 143.930001 113.450001) (width 0.25) (layer "F.Cu") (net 32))
 (segment (start 142.494 107.143339) (end 142.494 112.014) (width 0.25) (layer "F.Cu") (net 32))
 (segment (start 143.930001 113.450001) (end 144.78 114.3) (width 0.25) (layer "F.Cu") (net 32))
 (segment (start 141.119798 105.062031) (end 143.002 106.944233) (width 0.25) (layer "F.Cu") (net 33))
 (segment (start 143.002 109.982) (end 143.930001 110.910001) (width 0.25) (layer "F.Cu") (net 33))
 (segment (start 143.002 106.944233) (end 143.002 109.982) (width 0.25) (layer "F.Cu") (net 33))
 (segment (start 143.930001 110.910001) (end 144.78 111.76) (width 0.25) (layer "F.Cu") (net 33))
 (segment (start 143.51 106.745127) (end 143.51 107.95) (width 0.25) (layer "F.Cu") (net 34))
 (segment (start 141.473351 104.708478) (end 143.51 106.745127) (width 0.25) (layer "F.Cu") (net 34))
 (segment (start 143.51 107.95) (end 143.930001 108.370001) (width 0.25) (layer "F.Cu") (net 34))
 (segment (start 143.930001 108.370001) (end 144.78 109.22) (width 0.25) (layer "F.Cu") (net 34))
 (segment (start 144.151981 106.68) (end 144.78 106.68) (width 0.25) (layer "F.Cu") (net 35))
 (segment (start 141.826905 104.354924) (end 144.151981 106.68) (width 0.25) (layer "F.Cu") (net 35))
 (segment (start 143.803608 105.116392) (end 144.78 104.14) (width 0.25) (layer "F.Cu") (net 36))
 (segment (start 142.180458 104.001371) (end 143.295479 105.116392) (width 0.25) (layer "F.Cu") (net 36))
 (segment (start 143.295479 105.116392) (end 143.803608 105.116392) (width 0.25) (layer "F.Cu") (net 36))
 (segment (start 142.180458 101.738629) (end 143.335087 100.584) (width 0.25) (layer "F.Cu") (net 37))
 (segment (start 143.335087 100.584) (end 143.764 100.584) (width 0.25) (layer "F.Cu") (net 37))
 (segment (start 143.764 100.584) (end 144.78 101.6) (width 0.25) (layer "F.Cu") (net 37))
 (segment (start 141.826905 101.385076) (end 144.151981 99.06) (width 0.25) (layer "F.Cu") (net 38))
 (segment (start 144.151981 99.06) (end 144.78 99.06) (width 0.25) (layer "F.Cu") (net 38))
 (segment (start 141.473351 101.031522) (end 143.555099 98.949774) (width 0.25) (layer "F.Cu") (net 39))
 (segment (start 143.555099 98.949774) (end 143.555099 97.744901) (width 0.25) (layer "F.Cu") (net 39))
 (segment (start 143.930001 97.369999) (end 144.78 96.52) (width 0.25) (layer "F.Cu") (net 39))
 (segment (start 143.555099 97.744901) (end 143.930001 97.369999) (width 0.25) (layer "F.Cu") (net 39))
 (segment (start 141.119798 100.677969) (end 143.055189 98.742578) (width 0.25) (layer "F.Cu") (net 40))
 (segment (start 143.055189 98.742578) (end 143.055189 95.704811) (width 0.25) (layer "F.Cu") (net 40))
 (segment (start 143.930001 94.829999) (end 144.78 93.98) (width 0.25) (layer "F.Cu") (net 40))
 (segment (start 143.055189 95.704811) (end 143.930001 94.829999) (width 0.25) (layer "F.Cu") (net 40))
 (segment (start 142.555279 93.664721) (end 143.930001 92.289999) (width 0.25) (layer "F.Cu") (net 41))
 (segment (start 142.555279 98.535382) (end 142.555279 93.664721) (width 0.25) (layer "F.Cu") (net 41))
 (segment (start 140.766245 100.324416) (end 142.555279 98.535382) (width 0.25) (layer "F.Cu") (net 41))
 (segment (start 143.930001 92.289999) (end 144.78 91.44) (width 0.25) (layer "F.Cu") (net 41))
 (segment (start 142.055369 91.624631) (end 143.930001 89.749999) (width 0.25) (layer "F.Cu") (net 42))
 (segment (start 140.412691 99.970862) (end 142.055369 98.328184) (width 0.25) (layer "F.Cu") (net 42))
 (segment (start 142.055369 98.328184) (end 142.055369 91.624631) (width 0.25) (layer "F.Cu") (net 42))
 (segment (start 143.930001 89.749999) (end 144.78 88.9) (width 0.25) (layer "F.Cu") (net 42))
 (segment (start 143.930001 87.209999) (end 144.78 86.36) (width 0.25) (layer "F.Cu") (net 43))
 (segment (start 141.555459 98.120988) (end 141.555459 89.584541) (width 0.25) (layer "F.Cu") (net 43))
 (segment (start 141.555459 89.584541) (end 143.930001 87.209999) (width 0.25) (layer "F.Cu") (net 43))
 (segment (start 140.059138 99.617309) (end 141.555459 98.120988) (width 0.25) (layer "F.Cu") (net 43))
 (segment (start 141.055549 87.544451) (end 143.930001 84.669999) (width 0.25) (layer "F.Cu") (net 44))
 (segment (start 139.705584 99.263755) (end 141.055549 97.91379) (width 0.25) (layer "F.Cu") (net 44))
 (segment (start 143.930001 84.669999) (end 144.78 83.82) (width 0.25) (layer "F.Cu") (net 44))
 (segment (start 141.055549 97.91379) (end 141.055549 87.544451) (width 0.25) (layer "F.Cu") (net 44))
 (segment (start 139.352031 98.910202) (end 140.555639 97.706594) (width 0.25) (layer "F.Cu") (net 45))
 (segment (start 143.930001 82.129999) (end 144.78 81.28) (width 0.25) (layer "F.Cu") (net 45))
 (segment (start 140.555639 85.504361) (end 143.930001 82.129999) (width 0.25) (layer "F.Cu") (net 45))
 (segment (start 140.555639 97.706594) (end 140.555639 85.504361) (width 0.25) (layer "F.Cu") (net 45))
 (segment (start 140.055729 83.464271) (end 143.930001 79.589999) (width 0.25) (layer "F.Cu") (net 46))
 (segment (start 138.998478 98.556649) (end 140.055729 97.499398) (width 0.25) (layer "F.Cu") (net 46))
 (segment (start 143.930001 79.589999) (end 144.78 78.74) (width 0.25) (layer "F.Cu") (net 46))
 (segment (start 140.055729 97.499398) (end 140.055729 83.464271) (width 0.25) (layer "F.Cu") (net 46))
 (segment (start 139.555819 97.2922) (end 139.555819 81.424181) (width 0.25) (layer "F.Cu") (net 47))
 (segment (start 139.555819 81.424181) (end 143.930001 77.049999) (width 0.25) (layer "F.Cu") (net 47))
 (segment (start 138.644924 98.203095) (end 139.555819 97.2922) (width 0.25) (layer "F.Cu") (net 47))
 (segment (start 143.930001 77.049999) (end 144.78 76.2) (width 0.25) (layer "F.Cu") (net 47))
 (segment (start 139.055909 78.284091) (end 143.68 73.66) (width 0.25) (layer "F.Cu") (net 48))
 (segment (start 138.291371 97.849542) (end 139.055909 97.085004) (width 0.25) (layer "F.Cu") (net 48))
 (segment (start 139.055909 97.085004) (end 139.055909 78.284091) (width 0.25) (layer "F.Cu") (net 48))
 (segment (start 143.68 73.66) (end 144.78 73.66) (width 0.25) (layer "F.Cu") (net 48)))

